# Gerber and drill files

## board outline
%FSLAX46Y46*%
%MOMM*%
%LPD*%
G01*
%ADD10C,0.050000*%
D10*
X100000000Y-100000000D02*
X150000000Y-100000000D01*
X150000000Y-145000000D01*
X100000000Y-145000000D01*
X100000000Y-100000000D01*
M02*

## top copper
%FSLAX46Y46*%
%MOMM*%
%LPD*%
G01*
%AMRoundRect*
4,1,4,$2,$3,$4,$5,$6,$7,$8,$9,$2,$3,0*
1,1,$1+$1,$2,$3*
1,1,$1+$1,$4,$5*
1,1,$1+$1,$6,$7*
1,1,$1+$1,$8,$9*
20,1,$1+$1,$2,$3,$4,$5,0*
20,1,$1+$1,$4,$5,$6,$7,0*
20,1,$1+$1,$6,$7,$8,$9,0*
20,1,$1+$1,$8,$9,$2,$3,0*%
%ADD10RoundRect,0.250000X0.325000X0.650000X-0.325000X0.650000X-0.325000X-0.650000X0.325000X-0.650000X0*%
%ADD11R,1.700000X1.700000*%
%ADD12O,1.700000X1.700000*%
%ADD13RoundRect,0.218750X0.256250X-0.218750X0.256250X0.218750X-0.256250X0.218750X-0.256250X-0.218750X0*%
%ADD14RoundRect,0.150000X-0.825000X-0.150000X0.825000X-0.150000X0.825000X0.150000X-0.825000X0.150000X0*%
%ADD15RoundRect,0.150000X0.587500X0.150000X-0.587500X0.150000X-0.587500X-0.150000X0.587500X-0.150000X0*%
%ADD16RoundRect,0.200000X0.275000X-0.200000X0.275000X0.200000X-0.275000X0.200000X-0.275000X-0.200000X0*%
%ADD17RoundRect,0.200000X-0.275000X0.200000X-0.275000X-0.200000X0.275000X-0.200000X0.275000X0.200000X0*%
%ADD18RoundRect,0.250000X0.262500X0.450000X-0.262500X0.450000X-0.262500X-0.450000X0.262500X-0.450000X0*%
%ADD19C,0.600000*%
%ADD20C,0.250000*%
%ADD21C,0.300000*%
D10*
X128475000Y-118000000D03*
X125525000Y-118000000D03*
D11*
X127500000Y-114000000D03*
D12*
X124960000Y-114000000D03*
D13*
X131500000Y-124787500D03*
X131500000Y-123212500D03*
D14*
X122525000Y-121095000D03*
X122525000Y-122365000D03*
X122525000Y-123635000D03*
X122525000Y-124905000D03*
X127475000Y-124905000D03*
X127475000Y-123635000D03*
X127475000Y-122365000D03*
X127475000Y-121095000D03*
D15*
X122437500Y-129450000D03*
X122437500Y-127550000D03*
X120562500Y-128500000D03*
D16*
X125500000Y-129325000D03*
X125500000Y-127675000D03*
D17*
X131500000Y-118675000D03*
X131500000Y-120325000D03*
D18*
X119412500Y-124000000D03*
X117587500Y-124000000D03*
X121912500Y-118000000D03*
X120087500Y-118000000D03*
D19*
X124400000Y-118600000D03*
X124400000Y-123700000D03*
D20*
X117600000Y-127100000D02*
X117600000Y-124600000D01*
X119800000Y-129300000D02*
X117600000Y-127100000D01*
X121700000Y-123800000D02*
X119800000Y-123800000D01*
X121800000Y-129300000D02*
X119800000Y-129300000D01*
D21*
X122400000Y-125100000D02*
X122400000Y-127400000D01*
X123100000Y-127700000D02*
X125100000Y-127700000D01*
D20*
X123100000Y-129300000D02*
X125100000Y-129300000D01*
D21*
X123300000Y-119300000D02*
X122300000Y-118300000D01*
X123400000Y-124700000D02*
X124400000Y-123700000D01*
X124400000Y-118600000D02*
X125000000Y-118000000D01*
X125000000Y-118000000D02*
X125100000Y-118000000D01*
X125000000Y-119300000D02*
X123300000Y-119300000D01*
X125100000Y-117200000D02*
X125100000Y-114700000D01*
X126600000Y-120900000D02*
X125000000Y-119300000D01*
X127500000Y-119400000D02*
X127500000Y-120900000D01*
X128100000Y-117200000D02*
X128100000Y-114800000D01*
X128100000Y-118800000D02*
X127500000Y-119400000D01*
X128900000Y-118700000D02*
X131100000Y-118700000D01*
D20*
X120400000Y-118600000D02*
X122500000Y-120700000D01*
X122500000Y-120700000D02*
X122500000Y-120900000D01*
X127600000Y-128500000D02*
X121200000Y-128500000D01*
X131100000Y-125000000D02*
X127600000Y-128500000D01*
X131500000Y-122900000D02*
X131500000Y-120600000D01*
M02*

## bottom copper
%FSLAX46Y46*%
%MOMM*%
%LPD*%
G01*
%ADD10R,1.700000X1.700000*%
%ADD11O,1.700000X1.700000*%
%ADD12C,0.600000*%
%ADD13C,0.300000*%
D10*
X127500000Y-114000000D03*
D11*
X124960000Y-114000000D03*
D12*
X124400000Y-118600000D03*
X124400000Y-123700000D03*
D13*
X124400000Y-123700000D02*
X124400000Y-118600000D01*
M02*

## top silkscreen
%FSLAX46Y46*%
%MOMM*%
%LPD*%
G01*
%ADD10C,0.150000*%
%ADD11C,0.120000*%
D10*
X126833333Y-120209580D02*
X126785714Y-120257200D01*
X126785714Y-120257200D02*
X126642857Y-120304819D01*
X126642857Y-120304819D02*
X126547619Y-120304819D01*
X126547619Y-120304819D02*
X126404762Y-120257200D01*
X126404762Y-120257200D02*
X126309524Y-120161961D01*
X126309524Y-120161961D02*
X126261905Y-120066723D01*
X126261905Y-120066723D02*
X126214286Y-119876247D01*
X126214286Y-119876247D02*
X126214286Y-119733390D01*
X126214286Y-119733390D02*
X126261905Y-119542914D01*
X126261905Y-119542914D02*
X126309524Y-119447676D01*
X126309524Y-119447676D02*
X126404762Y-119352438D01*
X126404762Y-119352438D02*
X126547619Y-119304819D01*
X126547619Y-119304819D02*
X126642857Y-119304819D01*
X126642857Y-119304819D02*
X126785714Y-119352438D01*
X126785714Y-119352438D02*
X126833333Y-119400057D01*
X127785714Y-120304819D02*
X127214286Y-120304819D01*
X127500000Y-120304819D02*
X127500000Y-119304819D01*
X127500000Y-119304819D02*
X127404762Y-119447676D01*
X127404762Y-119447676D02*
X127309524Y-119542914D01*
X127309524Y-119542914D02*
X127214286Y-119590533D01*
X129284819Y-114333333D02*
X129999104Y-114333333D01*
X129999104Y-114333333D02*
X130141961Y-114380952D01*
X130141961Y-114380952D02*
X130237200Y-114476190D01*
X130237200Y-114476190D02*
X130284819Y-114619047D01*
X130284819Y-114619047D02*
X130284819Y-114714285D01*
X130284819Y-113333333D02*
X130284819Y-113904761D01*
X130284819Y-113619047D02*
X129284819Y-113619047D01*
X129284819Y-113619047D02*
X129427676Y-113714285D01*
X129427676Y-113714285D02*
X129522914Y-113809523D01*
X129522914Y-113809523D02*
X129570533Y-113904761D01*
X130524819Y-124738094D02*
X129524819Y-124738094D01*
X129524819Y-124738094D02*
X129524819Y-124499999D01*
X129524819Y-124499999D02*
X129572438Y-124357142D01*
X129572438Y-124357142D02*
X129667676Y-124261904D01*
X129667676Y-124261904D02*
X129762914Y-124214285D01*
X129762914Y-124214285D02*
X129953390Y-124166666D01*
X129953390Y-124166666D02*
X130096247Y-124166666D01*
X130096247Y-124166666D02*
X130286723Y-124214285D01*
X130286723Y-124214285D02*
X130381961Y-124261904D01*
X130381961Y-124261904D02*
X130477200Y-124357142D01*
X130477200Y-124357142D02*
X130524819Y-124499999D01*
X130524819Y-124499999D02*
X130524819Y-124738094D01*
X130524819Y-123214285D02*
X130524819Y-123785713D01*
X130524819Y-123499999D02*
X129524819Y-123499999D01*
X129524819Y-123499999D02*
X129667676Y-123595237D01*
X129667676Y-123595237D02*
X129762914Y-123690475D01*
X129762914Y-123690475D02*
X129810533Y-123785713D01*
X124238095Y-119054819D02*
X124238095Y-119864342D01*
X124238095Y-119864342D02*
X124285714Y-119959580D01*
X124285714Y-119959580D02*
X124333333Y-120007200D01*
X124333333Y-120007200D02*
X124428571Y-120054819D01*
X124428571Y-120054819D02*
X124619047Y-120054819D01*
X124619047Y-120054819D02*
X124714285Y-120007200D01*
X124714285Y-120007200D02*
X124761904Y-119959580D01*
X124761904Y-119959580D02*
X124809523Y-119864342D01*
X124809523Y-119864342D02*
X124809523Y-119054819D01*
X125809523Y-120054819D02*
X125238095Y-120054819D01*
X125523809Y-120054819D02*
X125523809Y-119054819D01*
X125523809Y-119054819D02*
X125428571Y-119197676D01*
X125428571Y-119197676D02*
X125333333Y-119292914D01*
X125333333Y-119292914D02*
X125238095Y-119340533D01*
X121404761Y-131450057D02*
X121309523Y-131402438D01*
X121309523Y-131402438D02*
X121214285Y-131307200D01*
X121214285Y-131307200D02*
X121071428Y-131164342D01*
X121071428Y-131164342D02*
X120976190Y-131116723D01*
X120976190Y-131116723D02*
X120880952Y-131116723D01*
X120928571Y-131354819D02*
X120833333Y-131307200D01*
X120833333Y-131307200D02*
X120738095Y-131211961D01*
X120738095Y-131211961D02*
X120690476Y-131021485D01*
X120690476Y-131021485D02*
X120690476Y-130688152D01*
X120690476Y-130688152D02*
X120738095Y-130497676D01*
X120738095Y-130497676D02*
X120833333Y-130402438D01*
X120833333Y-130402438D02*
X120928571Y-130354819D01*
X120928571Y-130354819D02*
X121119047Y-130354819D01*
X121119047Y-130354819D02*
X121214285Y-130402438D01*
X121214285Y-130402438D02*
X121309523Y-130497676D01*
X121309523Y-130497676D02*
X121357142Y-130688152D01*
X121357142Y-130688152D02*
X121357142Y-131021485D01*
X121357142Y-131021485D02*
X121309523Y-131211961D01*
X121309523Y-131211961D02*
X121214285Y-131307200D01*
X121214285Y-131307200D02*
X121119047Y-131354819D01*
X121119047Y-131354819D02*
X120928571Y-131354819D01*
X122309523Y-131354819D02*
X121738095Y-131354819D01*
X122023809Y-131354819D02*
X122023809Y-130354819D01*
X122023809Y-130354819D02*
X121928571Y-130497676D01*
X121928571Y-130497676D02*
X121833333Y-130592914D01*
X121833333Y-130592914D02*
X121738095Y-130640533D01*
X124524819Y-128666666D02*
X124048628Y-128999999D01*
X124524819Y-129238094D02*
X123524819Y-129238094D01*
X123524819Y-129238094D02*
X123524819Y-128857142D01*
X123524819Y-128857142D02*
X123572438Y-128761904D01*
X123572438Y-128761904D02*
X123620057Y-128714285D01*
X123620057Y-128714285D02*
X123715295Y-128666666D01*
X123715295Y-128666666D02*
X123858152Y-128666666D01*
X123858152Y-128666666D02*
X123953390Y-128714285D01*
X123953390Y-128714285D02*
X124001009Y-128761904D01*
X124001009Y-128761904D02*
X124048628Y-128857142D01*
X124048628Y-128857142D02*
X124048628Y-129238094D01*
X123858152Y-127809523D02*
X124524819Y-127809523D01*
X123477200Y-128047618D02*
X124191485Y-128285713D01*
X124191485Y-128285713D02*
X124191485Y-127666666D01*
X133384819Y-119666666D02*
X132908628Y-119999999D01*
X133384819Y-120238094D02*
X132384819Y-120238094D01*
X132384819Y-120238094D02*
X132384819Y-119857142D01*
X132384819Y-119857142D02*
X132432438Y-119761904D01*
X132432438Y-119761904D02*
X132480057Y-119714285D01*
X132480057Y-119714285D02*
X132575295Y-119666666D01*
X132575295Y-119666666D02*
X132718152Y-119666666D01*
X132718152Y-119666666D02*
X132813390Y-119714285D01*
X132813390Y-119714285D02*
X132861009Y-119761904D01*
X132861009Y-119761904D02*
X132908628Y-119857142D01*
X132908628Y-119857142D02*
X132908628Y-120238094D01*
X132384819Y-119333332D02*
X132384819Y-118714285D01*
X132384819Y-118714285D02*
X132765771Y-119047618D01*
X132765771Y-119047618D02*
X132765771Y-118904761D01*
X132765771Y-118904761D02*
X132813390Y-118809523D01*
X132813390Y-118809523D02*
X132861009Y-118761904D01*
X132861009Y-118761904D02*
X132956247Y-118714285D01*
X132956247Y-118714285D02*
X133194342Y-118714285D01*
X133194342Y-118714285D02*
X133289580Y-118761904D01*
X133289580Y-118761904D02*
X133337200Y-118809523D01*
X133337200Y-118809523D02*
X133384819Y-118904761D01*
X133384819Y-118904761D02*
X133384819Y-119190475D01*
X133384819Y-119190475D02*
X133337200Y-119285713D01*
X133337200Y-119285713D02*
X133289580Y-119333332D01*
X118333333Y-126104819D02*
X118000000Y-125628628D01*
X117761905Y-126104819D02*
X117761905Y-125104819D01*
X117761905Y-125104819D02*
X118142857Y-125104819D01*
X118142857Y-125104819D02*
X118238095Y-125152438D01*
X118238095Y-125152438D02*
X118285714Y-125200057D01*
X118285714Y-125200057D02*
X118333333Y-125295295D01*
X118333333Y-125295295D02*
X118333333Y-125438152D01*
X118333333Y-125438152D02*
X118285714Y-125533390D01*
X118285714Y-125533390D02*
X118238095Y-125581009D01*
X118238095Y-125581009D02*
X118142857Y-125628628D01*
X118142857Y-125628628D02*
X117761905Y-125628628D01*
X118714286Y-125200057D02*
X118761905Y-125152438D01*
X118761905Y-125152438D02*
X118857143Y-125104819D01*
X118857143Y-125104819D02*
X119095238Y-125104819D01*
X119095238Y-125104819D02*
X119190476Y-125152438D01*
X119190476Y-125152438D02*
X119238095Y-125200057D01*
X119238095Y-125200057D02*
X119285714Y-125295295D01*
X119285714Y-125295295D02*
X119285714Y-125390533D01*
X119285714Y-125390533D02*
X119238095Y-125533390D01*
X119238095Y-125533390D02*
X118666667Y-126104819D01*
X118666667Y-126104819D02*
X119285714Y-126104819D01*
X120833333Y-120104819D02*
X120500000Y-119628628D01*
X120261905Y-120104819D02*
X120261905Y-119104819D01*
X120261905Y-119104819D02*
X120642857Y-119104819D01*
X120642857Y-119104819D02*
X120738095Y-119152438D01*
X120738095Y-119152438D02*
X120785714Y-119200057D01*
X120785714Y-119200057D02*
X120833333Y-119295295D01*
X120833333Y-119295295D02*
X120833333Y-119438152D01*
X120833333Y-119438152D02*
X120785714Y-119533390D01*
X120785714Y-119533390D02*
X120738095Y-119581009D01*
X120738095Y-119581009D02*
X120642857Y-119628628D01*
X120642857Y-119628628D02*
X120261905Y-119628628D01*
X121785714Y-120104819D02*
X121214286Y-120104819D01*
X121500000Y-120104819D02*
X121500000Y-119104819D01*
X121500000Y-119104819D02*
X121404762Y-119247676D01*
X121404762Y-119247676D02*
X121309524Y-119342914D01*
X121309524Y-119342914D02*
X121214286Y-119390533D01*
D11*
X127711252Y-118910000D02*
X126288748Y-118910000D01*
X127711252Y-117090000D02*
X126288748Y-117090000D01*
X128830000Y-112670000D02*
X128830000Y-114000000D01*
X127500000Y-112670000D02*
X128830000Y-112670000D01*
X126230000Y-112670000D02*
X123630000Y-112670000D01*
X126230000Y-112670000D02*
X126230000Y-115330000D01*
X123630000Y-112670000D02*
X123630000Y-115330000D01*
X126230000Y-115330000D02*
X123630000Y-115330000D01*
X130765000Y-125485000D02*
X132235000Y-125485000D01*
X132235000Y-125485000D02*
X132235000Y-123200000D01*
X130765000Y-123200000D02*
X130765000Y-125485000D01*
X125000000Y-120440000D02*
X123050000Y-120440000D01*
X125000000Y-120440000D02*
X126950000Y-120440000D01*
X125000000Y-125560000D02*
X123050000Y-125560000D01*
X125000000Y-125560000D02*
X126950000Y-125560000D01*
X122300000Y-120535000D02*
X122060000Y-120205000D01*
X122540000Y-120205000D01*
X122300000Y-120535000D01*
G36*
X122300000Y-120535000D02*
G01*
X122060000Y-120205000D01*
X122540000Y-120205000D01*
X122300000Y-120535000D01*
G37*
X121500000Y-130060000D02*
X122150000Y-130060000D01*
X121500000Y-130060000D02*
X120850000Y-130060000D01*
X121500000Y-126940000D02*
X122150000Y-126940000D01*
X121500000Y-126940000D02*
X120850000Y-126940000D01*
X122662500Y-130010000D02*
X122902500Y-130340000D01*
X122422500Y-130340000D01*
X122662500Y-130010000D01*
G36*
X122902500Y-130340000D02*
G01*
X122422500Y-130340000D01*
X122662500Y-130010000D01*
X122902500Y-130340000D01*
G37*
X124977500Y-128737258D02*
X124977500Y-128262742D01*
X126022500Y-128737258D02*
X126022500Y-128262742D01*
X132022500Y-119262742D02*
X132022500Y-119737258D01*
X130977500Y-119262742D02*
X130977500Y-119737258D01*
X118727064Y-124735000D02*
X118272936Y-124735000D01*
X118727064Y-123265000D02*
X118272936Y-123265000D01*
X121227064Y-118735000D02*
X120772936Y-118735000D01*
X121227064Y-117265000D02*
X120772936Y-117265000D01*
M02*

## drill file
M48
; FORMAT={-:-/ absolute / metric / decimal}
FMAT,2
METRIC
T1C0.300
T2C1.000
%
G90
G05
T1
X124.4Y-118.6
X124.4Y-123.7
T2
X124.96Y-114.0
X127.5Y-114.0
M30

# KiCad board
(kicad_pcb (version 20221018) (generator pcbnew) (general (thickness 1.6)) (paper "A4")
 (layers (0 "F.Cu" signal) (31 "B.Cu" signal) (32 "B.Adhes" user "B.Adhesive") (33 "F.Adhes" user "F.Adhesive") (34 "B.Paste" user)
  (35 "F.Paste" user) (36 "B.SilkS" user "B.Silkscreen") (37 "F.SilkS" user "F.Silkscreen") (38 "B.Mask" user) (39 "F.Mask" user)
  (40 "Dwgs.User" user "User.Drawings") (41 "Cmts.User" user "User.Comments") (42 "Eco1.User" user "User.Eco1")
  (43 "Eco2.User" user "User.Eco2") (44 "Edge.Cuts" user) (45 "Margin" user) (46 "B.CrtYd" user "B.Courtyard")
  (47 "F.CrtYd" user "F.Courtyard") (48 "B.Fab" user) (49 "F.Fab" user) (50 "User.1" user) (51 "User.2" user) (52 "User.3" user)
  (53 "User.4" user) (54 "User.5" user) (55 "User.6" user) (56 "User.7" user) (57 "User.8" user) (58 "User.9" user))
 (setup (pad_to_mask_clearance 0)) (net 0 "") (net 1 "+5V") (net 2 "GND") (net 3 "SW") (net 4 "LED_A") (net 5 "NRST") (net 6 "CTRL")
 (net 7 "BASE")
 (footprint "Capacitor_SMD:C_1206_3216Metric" (layer "F.Cu") (at 127 118 180)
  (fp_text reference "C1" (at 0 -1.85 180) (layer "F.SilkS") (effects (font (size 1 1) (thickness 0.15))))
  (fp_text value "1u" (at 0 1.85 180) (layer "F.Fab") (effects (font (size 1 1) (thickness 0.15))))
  (fp_line (start -0.711252 -0.91) (end 0.711252 -0.91) (stroke (width 0.12) (type solid)) (layer "F.SilkS"))
  (fp_line (start -0.711252 0.91) (end 0.711252 0.91) (stroke (width 0.12) (type solid)) (layer "F.SilkS"))
  (pad "1" smd roundrect (at -1.475 0 180) (size 1.15 1.8) (layers "F.Cu" "F.Paste" "F.Mask") (roundrect_rratio 0.217391) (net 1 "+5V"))
  (pad "2" smd roundrect (at 1.475 0 180) (size 1.15 1.8) (layers "F.Cu" "F.Paste" "F.Mask") (roundrect_rratio 0.217391) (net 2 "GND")))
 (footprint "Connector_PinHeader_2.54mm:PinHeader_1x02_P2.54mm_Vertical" (layer "F.Cu") (at 127.5 114 -90)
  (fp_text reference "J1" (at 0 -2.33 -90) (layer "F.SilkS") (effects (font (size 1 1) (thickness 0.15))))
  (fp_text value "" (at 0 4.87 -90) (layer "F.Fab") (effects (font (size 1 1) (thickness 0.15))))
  (fp_line (start -1.33 -1.33) (end 0 -1.33) (stroke (width 0.12) (type solid)) (layer "F.SilkS"))
  (fp_line (start -1.33 0) (end -1.33 -1.33) (stroke (width 0.12) (type solid)) (layer "F.SilkS"))
  (fp_line (start -1.33 1.27) (end -1.33 3.87) (stroke (width 0.12) (type solid)) (layer "F.SilkS"))
  (fp_line (start -1.33 1.27) (end 1.33 1.27) (stroke (width 0.12) (type solid)) (layer "F.SilkS"))
  (fp_line (start -1.33 3.87) (end 1.33 3.87) (stroke (width 0.12) (type solid)) (layer "F.SilkS"))
  (fp_line (start 1.33 1.27) (end 1.33 3.87) (stroke (width 0.12) (type solid)) (layer "F.SilkS"))
  (pad "1" thru_hole rect (at 0 0 270) (size 1.7 1.7) (drill 1) (layers "*.Cu" "*.Mask") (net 1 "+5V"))
  (pad "2" thru_hole oval (at 0 2.54 270) (size 1.7 1.7) (drill 1) (layers "*.Cu" "*.Mask") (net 2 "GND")))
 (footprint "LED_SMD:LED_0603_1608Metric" (layer "F.Cu") (at 131.5 124 90)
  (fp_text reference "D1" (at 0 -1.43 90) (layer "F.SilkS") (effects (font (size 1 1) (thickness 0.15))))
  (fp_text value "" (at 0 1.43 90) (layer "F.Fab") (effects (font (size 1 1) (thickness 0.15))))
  (fp_line (start -1.485 -0.735) (end -1.485 0.735) (stroke (width 0.12) (type solid)) (layer "F.SilkS"))
  (fp_line (start -1.485 0.735) (end 0.8 0.735) (stroke (width 0.12) (type solid)) (layer "F.SilkS"))
  (fp_line (start 0.8 -0.735) (end -1.485 -0.735) (stroke (width 0.12) (type solid)) (layer "F.SilkS"))
  (pad "1" smd roundrect (at -0.7875 0 90) (size 0.875 0.95) (layers "F.Cu" "F.Paste" "F.Mask") (roundrect_rratio 0.25) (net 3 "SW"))
  (pad "2" smd roundrect (at 0.7875 0 90) (size 0.875 0.95) (layers "F.Cu" "F.Paste" "F.Mask") (roundrect_rratio 0.25) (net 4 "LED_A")))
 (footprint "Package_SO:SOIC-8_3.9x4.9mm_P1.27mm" (layer "F.Cu") (at 125 123)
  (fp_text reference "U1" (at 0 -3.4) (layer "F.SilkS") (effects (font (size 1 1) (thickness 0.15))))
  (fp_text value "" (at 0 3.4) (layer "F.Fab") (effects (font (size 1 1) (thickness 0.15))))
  (fp_line (start 0 -2.56) (end -1.95 -2.56) (stroke (width 0.12) (type solid)) (layer "F.SilkS"))
  (fp_line (start 0 -2.56) (end 1.95 -2.56) (stroke (width 0.12) (type solid)) (layer "F.SilkS"))
  (fp_line (start 0 2.56) (end -1.95 2.56) (stroke (width 0.12) (type solid)) (layer "F.SilkS"))
  (fp_line (start 0 2.56) (end 1.95 2.56) (stroke (width 0.12) (type solid)) (layer "F.SilkS"))
  (fp_poly
   (pts (xy -2.7 -2.465) (xy -2.94 -2.795) (xy -2.46 -2.795) (xy -2.7 -2.465)) (stroke (width 0.12) (type solid)) (fill solid)
   (layer "F.SilkS"))
  (pad "1" smd roundrect (at -2.475 -1.905) (size 1.95 0.6) (layers "F.Cu" "F.Paste" "F.Mask") (roundrect_rratio 0.25) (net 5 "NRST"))
  (pad "2" smd roundrect (at -2.475 -0.635) (size 1.95 0.6) (layers "F.Cu" "F.Paste" "F.Mask") (roundrect_rratio 0.25))
  (pad "3" smd roundrect (at -2.475 0.635) (size 1.95 0.6) (layers "F.Cu" "F.Paste" "F.Mask") (roundrect_rratio 0.25) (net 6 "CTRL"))
  (pad "4" smd roundrect (at -2.475 1.905) (size 1.95 0.6) (layers "F.Cu" "F.Paste" "F.Mask") (roundrect_rratio 0.25) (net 2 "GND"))
  (pad "5" smd roundrect (at 2.475 1.905) (size 1.95 0.6) (layers "F.Cu" "F.Paste" "F.Mask") (roundrect_rratio 0.25))
  (pad "6" smd roundrect (at 2.475 0.635) (size 1.95 0.6) (layers "F.Cu" "F.Paste" "F.Mask") (roundrect_rratio 0.25))
  (pad "7" smd roundrect (at 2.475 -0.635) (size 1.95 0.6) (layers "F.Cu" "F.Paste" "F.Mask") (roundrect_rratio 0.25))
  (pad "8" smd roundrect (at 2.475 -1.905) (size 1.95 0.6) (layers "F.Cu" "F.Paste" "F.Mask") (roundrect_rratio 0.25) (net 1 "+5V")))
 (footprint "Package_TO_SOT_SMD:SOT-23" (layer "F.Cu") (at 121.5 128.5 180)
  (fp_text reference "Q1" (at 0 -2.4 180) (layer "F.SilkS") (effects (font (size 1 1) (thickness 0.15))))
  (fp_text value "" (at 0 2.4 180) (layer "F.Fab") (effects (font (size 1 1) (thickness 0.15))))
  (fp_line (start 0 -1.56) (end -0.65 -1.56) (stroke (width 0.12) (type solid)) (layer "F.SilkS"))
  (fp_line (start 0 -1.56) (end 0.65 -1.56) (stroke (width 0.12) (type solid)) (layer "F.SilkS"))
  (fp_line (start 0 1.56) (end -0.65 1.56) (stroke (width 0.12) (type solid)) (layer "F.SilkS"))
  (fp_line (start 0 1.56) (end 0.65 1.56) (stroke (width 0.12) (type solid)) (layer "F.SilkS"))
  (fp_poly
   (pts (xy -1.1625 -1.51) (xy -1.4025 -1.84) (xy -0.9225 -1.84) (xy -1.1625 -1.51)) (stroke (width 0.12) (type solid)) (fill solid)
   (layer "F.SilkS"))
  (pad "1" smd roundrect (at -0.9375 -0.95 180) (size 1.475 0.6) (layers "F.Cu" "F.Paste" "F.Mask") (roundrect_rratio 0.25) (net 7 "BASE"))
  (pad "2" smd roundrect (at -0.9375 0.95 180) (size 1.475 0.6) (layers "F.Cu" "F.Paste" "F.Mask") (roundrect_rratio 0.25) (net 2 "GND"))
  (pad "3" smd roundrect (at 0.9375 0 180) (size 1.475 0.6) (layers "F.Cu" "F.Paste" "F.Mask") (roundrect_rratio 0.25) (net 3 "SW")))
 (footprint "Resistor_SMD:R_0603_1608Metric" (layer "F.Cu") (at 125.5 128.5 90)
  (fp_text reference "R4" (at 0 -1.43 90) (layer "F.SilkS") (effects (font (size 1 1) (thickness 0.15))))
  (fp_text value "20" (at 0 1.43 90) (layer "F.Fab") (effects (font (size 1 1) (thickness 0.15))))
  (fp_line (start -0.237258 -0.5225) (end 0.237258 -0.5225) (stroke (width 0.12) (type solid)) (layer "F.SilkS"))
  (fp_line (start -0.237258 0.5225) (end 0.237258 0.5225) (stroke (width 0.12) (type solid)) (layer "F.SilkS"))
  (pad "1" smd roundrect (at -0.825 0 90) (size 0.8 0.95) (layers "F.Cu" "F.Paste" "F.Mask") (roundrect_rratio 0.25) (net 7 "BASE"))
  (pad "2" smd roundrect (at 0.825 0 90) (size 0.8 0.95) (layers "F.Cu" "F.Paste" "F.Mask") (roundrect_rratio 0.25) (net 2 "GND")))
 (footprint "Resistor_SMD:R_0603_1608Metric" (layer "F.Cu") (at 131.5 119.5 -90)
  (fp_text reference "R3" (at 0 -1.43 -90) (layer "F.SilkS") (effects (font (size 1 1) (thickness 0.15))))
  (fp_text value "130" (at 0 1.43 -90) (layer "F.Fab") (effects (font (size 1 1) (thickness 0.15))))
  (fp_line (start -0.237258 -0.5225) (end 0.237258 -0.5225) (stroke (width 0.12) (type solid)) (layer "F.SilkS"))
  (fp_line (start -0.237258 0.5225) (end 0.237258 0.5225) (stroke (width 0.12) (type solid)) (layer "F.SilkS"))
  (pad "1" smd roundrect (at -0.825 0 270) (size 0.8 0.95) (layers "F.Cu" "F.Paste" "F.Mask") (roundrect_rratio 0.25) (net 1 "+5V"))
  (pad "2" smd roundrect (at 0.825 0 270) (size 0.8 0.95) (layers "F.Cu" "F.Paste" "F.Mask") (roundrect_rratio 0.25) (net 4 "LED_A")))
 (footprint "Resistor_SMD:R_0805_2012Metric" (layer "F.Cu") (at 118.5 124 180)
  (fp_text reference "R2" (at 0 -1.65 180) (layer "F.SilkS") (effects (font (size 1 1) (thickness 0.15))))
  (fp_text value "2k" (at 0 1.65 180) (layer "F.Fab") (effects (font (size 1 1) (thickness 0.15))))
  (fp_line (start -0.227064 -0.735) (end 0.227064 -0.735) (stroke (width 0.12) (type solid)) (layer "F.SilkS"))
  (fp_line (start -0.227064 0.735) (end 0.227064 0.735) (stroke (width 0.12) (type solid)) (layer "F.SilkS"))
  (pad "1" smd roundrect (at -0.9125 0 180) (size 1.025 1.4) (layers "F.Cu" "F.Paste" "F.Mask") (roundrect_rratio 0.243902) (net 6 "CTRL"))
  (pad "2" smd roundrect (at 0.9125 0 180) (size 1.025 1.4) (layers "F.Cu" "F.Paste" "F.Mask") (roundrect_rratio 0.243902) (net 7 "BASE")))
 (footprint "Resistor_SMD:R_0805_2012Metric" (layer "F.Cu") (at 121 118 180)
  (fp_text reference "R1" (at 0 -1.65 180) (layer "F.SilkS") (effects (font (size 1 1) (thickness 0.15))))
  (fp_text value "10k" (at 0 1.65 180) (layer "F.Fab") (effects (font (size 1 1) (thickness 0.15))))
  (fp_line (start -0.227064 -0.735) (end 0.227064 -0.735) (stroke (width 0.12) (type solid)) (layer "F.SilkS"))
  (fp_line (start -0.227064 0.735) (end 0.227064 0.735) (stroke (width 0.12) (type solid)) (layer "F.SilkS"))
  (pad "1" smd roundrect (at -0.9125 0 180) (size 1.025 1.4) (layers "F.Cu" "F.Paste" "F.Mask") (roundrect_rratio 0.243902) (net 1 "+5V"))
  (pad "2" smd roundrect (at 0.9125 0 180) (size 1.025 1.4) (layers "F.Cu" "F.Paste" "F.Mask") (roundrect_rratio 0.243902) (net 5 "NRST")))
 (gr_rect (start 100 100) (end 150 145) (stroke (width 0.05) (type default)) (fill none) (layer "Edge.Cuts"))
 (segment (start 117.6 127.1) (end 117.6 124.6) (width 0.25) (layer "F.Cu") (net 7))
 (segment (start 119.8 129.3) (end 117.6 127.1) (width 0.25) (layer "F.Cu") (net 7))
 (segment (start 121.7 123.8) (end 119.8 123.8) (width 0.25) (layer "F.Cu") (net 6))
 (segment (start 121.8 129.3) (end 119.8 129.3) (width 0.25) (layer "F.Cu") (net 7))
 (segment (start 122.4 125.1) (end 122.4 127.4) (width 0.3) (layer "F.Cu") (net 2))
 (segment (start 123.1 127.7) (end 125.1 127.7) (width 0.3) (layer "F.Cu") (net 2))
 (segment (start 123.1 129.3) (end 125.1 129.3) (width 0.25) (layer "F.Cu") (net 7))
 (segment (start 123.3 119.3) (end 122.3 118.3) (width 0.3) (layer "F.Cu") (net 1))
 (segment (start 123.4 124.7) (end 124.4 123.7) (width 0.3) (layer "F.Cu") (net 2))
 (segment (start 124.4 118.6) (end 125 118) (width 0.3) (layer "F.Cu") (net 2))
 (segment (start 125 118) (end 125.1 118) (width 0.3) (layer "F.Cu") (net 2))
 (segment (start 125 119.3) (end 123.3 119.3) (width 0.3) (layer "F.Cu") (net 1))
 (segment (start 125.1 117.2) (end 125.1 114.7) (width 0.3) (layer "F.Cu") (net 2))
 (segment (start 126.6 120.9) (end 125 119.3) (width 0.3) (layer "F.Cu") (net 1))
 (segment (start 127.5 119.4) (end 127.5 120.9) (width 0.3) (layer "F.Cu") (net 1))
 (segment (start 128.1 117.2) (end 128.1 114.8) (width 0.3) (layer "F.Cu") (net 1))
 (segment (start 128.1 118.8) (end 127.5 119.4) (width 0.3) (layer "F.Cu") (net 1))
 (segment (start 128.9 118.7) (end 131.1 118.7) (width 0.3) (layer "F.Cu") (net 1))
 (via (at 124.4 118.6) (size 0.6) (drill 0.3) (layers "F.Cu" "B.Cu") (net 2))
 (via (at 124.4 123.7) (size 0.6) (drill 0.3) (layers "F.Cu" "B.Cu") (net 2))
 (segment (start 120.4 118.6) (end 122.5 120.7) (width 0.25) (layer "F.Cu") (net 5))
 (segment (start 122.5 120.7) (end 122.5 120.9) (width 0.25) (layer "F.Cu") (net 5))
 (segment (start 124.4 123.7) (end 124.4 118.6) (width 0.3) (layer "B.Cu") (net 2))
 (segment (start 127.6 128.5) (end 121.2 128.5) (width 0.25) (layer "F.Cu") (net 3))
 (segment (start 131.1 125) (end 127.6 128.5) (width 0.25) (layer "F.Cu") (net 3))
 (segment (start 131.5 122.9) (end 131.5 120.6) (width 0.25) (layer "F.Cu") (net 4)))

